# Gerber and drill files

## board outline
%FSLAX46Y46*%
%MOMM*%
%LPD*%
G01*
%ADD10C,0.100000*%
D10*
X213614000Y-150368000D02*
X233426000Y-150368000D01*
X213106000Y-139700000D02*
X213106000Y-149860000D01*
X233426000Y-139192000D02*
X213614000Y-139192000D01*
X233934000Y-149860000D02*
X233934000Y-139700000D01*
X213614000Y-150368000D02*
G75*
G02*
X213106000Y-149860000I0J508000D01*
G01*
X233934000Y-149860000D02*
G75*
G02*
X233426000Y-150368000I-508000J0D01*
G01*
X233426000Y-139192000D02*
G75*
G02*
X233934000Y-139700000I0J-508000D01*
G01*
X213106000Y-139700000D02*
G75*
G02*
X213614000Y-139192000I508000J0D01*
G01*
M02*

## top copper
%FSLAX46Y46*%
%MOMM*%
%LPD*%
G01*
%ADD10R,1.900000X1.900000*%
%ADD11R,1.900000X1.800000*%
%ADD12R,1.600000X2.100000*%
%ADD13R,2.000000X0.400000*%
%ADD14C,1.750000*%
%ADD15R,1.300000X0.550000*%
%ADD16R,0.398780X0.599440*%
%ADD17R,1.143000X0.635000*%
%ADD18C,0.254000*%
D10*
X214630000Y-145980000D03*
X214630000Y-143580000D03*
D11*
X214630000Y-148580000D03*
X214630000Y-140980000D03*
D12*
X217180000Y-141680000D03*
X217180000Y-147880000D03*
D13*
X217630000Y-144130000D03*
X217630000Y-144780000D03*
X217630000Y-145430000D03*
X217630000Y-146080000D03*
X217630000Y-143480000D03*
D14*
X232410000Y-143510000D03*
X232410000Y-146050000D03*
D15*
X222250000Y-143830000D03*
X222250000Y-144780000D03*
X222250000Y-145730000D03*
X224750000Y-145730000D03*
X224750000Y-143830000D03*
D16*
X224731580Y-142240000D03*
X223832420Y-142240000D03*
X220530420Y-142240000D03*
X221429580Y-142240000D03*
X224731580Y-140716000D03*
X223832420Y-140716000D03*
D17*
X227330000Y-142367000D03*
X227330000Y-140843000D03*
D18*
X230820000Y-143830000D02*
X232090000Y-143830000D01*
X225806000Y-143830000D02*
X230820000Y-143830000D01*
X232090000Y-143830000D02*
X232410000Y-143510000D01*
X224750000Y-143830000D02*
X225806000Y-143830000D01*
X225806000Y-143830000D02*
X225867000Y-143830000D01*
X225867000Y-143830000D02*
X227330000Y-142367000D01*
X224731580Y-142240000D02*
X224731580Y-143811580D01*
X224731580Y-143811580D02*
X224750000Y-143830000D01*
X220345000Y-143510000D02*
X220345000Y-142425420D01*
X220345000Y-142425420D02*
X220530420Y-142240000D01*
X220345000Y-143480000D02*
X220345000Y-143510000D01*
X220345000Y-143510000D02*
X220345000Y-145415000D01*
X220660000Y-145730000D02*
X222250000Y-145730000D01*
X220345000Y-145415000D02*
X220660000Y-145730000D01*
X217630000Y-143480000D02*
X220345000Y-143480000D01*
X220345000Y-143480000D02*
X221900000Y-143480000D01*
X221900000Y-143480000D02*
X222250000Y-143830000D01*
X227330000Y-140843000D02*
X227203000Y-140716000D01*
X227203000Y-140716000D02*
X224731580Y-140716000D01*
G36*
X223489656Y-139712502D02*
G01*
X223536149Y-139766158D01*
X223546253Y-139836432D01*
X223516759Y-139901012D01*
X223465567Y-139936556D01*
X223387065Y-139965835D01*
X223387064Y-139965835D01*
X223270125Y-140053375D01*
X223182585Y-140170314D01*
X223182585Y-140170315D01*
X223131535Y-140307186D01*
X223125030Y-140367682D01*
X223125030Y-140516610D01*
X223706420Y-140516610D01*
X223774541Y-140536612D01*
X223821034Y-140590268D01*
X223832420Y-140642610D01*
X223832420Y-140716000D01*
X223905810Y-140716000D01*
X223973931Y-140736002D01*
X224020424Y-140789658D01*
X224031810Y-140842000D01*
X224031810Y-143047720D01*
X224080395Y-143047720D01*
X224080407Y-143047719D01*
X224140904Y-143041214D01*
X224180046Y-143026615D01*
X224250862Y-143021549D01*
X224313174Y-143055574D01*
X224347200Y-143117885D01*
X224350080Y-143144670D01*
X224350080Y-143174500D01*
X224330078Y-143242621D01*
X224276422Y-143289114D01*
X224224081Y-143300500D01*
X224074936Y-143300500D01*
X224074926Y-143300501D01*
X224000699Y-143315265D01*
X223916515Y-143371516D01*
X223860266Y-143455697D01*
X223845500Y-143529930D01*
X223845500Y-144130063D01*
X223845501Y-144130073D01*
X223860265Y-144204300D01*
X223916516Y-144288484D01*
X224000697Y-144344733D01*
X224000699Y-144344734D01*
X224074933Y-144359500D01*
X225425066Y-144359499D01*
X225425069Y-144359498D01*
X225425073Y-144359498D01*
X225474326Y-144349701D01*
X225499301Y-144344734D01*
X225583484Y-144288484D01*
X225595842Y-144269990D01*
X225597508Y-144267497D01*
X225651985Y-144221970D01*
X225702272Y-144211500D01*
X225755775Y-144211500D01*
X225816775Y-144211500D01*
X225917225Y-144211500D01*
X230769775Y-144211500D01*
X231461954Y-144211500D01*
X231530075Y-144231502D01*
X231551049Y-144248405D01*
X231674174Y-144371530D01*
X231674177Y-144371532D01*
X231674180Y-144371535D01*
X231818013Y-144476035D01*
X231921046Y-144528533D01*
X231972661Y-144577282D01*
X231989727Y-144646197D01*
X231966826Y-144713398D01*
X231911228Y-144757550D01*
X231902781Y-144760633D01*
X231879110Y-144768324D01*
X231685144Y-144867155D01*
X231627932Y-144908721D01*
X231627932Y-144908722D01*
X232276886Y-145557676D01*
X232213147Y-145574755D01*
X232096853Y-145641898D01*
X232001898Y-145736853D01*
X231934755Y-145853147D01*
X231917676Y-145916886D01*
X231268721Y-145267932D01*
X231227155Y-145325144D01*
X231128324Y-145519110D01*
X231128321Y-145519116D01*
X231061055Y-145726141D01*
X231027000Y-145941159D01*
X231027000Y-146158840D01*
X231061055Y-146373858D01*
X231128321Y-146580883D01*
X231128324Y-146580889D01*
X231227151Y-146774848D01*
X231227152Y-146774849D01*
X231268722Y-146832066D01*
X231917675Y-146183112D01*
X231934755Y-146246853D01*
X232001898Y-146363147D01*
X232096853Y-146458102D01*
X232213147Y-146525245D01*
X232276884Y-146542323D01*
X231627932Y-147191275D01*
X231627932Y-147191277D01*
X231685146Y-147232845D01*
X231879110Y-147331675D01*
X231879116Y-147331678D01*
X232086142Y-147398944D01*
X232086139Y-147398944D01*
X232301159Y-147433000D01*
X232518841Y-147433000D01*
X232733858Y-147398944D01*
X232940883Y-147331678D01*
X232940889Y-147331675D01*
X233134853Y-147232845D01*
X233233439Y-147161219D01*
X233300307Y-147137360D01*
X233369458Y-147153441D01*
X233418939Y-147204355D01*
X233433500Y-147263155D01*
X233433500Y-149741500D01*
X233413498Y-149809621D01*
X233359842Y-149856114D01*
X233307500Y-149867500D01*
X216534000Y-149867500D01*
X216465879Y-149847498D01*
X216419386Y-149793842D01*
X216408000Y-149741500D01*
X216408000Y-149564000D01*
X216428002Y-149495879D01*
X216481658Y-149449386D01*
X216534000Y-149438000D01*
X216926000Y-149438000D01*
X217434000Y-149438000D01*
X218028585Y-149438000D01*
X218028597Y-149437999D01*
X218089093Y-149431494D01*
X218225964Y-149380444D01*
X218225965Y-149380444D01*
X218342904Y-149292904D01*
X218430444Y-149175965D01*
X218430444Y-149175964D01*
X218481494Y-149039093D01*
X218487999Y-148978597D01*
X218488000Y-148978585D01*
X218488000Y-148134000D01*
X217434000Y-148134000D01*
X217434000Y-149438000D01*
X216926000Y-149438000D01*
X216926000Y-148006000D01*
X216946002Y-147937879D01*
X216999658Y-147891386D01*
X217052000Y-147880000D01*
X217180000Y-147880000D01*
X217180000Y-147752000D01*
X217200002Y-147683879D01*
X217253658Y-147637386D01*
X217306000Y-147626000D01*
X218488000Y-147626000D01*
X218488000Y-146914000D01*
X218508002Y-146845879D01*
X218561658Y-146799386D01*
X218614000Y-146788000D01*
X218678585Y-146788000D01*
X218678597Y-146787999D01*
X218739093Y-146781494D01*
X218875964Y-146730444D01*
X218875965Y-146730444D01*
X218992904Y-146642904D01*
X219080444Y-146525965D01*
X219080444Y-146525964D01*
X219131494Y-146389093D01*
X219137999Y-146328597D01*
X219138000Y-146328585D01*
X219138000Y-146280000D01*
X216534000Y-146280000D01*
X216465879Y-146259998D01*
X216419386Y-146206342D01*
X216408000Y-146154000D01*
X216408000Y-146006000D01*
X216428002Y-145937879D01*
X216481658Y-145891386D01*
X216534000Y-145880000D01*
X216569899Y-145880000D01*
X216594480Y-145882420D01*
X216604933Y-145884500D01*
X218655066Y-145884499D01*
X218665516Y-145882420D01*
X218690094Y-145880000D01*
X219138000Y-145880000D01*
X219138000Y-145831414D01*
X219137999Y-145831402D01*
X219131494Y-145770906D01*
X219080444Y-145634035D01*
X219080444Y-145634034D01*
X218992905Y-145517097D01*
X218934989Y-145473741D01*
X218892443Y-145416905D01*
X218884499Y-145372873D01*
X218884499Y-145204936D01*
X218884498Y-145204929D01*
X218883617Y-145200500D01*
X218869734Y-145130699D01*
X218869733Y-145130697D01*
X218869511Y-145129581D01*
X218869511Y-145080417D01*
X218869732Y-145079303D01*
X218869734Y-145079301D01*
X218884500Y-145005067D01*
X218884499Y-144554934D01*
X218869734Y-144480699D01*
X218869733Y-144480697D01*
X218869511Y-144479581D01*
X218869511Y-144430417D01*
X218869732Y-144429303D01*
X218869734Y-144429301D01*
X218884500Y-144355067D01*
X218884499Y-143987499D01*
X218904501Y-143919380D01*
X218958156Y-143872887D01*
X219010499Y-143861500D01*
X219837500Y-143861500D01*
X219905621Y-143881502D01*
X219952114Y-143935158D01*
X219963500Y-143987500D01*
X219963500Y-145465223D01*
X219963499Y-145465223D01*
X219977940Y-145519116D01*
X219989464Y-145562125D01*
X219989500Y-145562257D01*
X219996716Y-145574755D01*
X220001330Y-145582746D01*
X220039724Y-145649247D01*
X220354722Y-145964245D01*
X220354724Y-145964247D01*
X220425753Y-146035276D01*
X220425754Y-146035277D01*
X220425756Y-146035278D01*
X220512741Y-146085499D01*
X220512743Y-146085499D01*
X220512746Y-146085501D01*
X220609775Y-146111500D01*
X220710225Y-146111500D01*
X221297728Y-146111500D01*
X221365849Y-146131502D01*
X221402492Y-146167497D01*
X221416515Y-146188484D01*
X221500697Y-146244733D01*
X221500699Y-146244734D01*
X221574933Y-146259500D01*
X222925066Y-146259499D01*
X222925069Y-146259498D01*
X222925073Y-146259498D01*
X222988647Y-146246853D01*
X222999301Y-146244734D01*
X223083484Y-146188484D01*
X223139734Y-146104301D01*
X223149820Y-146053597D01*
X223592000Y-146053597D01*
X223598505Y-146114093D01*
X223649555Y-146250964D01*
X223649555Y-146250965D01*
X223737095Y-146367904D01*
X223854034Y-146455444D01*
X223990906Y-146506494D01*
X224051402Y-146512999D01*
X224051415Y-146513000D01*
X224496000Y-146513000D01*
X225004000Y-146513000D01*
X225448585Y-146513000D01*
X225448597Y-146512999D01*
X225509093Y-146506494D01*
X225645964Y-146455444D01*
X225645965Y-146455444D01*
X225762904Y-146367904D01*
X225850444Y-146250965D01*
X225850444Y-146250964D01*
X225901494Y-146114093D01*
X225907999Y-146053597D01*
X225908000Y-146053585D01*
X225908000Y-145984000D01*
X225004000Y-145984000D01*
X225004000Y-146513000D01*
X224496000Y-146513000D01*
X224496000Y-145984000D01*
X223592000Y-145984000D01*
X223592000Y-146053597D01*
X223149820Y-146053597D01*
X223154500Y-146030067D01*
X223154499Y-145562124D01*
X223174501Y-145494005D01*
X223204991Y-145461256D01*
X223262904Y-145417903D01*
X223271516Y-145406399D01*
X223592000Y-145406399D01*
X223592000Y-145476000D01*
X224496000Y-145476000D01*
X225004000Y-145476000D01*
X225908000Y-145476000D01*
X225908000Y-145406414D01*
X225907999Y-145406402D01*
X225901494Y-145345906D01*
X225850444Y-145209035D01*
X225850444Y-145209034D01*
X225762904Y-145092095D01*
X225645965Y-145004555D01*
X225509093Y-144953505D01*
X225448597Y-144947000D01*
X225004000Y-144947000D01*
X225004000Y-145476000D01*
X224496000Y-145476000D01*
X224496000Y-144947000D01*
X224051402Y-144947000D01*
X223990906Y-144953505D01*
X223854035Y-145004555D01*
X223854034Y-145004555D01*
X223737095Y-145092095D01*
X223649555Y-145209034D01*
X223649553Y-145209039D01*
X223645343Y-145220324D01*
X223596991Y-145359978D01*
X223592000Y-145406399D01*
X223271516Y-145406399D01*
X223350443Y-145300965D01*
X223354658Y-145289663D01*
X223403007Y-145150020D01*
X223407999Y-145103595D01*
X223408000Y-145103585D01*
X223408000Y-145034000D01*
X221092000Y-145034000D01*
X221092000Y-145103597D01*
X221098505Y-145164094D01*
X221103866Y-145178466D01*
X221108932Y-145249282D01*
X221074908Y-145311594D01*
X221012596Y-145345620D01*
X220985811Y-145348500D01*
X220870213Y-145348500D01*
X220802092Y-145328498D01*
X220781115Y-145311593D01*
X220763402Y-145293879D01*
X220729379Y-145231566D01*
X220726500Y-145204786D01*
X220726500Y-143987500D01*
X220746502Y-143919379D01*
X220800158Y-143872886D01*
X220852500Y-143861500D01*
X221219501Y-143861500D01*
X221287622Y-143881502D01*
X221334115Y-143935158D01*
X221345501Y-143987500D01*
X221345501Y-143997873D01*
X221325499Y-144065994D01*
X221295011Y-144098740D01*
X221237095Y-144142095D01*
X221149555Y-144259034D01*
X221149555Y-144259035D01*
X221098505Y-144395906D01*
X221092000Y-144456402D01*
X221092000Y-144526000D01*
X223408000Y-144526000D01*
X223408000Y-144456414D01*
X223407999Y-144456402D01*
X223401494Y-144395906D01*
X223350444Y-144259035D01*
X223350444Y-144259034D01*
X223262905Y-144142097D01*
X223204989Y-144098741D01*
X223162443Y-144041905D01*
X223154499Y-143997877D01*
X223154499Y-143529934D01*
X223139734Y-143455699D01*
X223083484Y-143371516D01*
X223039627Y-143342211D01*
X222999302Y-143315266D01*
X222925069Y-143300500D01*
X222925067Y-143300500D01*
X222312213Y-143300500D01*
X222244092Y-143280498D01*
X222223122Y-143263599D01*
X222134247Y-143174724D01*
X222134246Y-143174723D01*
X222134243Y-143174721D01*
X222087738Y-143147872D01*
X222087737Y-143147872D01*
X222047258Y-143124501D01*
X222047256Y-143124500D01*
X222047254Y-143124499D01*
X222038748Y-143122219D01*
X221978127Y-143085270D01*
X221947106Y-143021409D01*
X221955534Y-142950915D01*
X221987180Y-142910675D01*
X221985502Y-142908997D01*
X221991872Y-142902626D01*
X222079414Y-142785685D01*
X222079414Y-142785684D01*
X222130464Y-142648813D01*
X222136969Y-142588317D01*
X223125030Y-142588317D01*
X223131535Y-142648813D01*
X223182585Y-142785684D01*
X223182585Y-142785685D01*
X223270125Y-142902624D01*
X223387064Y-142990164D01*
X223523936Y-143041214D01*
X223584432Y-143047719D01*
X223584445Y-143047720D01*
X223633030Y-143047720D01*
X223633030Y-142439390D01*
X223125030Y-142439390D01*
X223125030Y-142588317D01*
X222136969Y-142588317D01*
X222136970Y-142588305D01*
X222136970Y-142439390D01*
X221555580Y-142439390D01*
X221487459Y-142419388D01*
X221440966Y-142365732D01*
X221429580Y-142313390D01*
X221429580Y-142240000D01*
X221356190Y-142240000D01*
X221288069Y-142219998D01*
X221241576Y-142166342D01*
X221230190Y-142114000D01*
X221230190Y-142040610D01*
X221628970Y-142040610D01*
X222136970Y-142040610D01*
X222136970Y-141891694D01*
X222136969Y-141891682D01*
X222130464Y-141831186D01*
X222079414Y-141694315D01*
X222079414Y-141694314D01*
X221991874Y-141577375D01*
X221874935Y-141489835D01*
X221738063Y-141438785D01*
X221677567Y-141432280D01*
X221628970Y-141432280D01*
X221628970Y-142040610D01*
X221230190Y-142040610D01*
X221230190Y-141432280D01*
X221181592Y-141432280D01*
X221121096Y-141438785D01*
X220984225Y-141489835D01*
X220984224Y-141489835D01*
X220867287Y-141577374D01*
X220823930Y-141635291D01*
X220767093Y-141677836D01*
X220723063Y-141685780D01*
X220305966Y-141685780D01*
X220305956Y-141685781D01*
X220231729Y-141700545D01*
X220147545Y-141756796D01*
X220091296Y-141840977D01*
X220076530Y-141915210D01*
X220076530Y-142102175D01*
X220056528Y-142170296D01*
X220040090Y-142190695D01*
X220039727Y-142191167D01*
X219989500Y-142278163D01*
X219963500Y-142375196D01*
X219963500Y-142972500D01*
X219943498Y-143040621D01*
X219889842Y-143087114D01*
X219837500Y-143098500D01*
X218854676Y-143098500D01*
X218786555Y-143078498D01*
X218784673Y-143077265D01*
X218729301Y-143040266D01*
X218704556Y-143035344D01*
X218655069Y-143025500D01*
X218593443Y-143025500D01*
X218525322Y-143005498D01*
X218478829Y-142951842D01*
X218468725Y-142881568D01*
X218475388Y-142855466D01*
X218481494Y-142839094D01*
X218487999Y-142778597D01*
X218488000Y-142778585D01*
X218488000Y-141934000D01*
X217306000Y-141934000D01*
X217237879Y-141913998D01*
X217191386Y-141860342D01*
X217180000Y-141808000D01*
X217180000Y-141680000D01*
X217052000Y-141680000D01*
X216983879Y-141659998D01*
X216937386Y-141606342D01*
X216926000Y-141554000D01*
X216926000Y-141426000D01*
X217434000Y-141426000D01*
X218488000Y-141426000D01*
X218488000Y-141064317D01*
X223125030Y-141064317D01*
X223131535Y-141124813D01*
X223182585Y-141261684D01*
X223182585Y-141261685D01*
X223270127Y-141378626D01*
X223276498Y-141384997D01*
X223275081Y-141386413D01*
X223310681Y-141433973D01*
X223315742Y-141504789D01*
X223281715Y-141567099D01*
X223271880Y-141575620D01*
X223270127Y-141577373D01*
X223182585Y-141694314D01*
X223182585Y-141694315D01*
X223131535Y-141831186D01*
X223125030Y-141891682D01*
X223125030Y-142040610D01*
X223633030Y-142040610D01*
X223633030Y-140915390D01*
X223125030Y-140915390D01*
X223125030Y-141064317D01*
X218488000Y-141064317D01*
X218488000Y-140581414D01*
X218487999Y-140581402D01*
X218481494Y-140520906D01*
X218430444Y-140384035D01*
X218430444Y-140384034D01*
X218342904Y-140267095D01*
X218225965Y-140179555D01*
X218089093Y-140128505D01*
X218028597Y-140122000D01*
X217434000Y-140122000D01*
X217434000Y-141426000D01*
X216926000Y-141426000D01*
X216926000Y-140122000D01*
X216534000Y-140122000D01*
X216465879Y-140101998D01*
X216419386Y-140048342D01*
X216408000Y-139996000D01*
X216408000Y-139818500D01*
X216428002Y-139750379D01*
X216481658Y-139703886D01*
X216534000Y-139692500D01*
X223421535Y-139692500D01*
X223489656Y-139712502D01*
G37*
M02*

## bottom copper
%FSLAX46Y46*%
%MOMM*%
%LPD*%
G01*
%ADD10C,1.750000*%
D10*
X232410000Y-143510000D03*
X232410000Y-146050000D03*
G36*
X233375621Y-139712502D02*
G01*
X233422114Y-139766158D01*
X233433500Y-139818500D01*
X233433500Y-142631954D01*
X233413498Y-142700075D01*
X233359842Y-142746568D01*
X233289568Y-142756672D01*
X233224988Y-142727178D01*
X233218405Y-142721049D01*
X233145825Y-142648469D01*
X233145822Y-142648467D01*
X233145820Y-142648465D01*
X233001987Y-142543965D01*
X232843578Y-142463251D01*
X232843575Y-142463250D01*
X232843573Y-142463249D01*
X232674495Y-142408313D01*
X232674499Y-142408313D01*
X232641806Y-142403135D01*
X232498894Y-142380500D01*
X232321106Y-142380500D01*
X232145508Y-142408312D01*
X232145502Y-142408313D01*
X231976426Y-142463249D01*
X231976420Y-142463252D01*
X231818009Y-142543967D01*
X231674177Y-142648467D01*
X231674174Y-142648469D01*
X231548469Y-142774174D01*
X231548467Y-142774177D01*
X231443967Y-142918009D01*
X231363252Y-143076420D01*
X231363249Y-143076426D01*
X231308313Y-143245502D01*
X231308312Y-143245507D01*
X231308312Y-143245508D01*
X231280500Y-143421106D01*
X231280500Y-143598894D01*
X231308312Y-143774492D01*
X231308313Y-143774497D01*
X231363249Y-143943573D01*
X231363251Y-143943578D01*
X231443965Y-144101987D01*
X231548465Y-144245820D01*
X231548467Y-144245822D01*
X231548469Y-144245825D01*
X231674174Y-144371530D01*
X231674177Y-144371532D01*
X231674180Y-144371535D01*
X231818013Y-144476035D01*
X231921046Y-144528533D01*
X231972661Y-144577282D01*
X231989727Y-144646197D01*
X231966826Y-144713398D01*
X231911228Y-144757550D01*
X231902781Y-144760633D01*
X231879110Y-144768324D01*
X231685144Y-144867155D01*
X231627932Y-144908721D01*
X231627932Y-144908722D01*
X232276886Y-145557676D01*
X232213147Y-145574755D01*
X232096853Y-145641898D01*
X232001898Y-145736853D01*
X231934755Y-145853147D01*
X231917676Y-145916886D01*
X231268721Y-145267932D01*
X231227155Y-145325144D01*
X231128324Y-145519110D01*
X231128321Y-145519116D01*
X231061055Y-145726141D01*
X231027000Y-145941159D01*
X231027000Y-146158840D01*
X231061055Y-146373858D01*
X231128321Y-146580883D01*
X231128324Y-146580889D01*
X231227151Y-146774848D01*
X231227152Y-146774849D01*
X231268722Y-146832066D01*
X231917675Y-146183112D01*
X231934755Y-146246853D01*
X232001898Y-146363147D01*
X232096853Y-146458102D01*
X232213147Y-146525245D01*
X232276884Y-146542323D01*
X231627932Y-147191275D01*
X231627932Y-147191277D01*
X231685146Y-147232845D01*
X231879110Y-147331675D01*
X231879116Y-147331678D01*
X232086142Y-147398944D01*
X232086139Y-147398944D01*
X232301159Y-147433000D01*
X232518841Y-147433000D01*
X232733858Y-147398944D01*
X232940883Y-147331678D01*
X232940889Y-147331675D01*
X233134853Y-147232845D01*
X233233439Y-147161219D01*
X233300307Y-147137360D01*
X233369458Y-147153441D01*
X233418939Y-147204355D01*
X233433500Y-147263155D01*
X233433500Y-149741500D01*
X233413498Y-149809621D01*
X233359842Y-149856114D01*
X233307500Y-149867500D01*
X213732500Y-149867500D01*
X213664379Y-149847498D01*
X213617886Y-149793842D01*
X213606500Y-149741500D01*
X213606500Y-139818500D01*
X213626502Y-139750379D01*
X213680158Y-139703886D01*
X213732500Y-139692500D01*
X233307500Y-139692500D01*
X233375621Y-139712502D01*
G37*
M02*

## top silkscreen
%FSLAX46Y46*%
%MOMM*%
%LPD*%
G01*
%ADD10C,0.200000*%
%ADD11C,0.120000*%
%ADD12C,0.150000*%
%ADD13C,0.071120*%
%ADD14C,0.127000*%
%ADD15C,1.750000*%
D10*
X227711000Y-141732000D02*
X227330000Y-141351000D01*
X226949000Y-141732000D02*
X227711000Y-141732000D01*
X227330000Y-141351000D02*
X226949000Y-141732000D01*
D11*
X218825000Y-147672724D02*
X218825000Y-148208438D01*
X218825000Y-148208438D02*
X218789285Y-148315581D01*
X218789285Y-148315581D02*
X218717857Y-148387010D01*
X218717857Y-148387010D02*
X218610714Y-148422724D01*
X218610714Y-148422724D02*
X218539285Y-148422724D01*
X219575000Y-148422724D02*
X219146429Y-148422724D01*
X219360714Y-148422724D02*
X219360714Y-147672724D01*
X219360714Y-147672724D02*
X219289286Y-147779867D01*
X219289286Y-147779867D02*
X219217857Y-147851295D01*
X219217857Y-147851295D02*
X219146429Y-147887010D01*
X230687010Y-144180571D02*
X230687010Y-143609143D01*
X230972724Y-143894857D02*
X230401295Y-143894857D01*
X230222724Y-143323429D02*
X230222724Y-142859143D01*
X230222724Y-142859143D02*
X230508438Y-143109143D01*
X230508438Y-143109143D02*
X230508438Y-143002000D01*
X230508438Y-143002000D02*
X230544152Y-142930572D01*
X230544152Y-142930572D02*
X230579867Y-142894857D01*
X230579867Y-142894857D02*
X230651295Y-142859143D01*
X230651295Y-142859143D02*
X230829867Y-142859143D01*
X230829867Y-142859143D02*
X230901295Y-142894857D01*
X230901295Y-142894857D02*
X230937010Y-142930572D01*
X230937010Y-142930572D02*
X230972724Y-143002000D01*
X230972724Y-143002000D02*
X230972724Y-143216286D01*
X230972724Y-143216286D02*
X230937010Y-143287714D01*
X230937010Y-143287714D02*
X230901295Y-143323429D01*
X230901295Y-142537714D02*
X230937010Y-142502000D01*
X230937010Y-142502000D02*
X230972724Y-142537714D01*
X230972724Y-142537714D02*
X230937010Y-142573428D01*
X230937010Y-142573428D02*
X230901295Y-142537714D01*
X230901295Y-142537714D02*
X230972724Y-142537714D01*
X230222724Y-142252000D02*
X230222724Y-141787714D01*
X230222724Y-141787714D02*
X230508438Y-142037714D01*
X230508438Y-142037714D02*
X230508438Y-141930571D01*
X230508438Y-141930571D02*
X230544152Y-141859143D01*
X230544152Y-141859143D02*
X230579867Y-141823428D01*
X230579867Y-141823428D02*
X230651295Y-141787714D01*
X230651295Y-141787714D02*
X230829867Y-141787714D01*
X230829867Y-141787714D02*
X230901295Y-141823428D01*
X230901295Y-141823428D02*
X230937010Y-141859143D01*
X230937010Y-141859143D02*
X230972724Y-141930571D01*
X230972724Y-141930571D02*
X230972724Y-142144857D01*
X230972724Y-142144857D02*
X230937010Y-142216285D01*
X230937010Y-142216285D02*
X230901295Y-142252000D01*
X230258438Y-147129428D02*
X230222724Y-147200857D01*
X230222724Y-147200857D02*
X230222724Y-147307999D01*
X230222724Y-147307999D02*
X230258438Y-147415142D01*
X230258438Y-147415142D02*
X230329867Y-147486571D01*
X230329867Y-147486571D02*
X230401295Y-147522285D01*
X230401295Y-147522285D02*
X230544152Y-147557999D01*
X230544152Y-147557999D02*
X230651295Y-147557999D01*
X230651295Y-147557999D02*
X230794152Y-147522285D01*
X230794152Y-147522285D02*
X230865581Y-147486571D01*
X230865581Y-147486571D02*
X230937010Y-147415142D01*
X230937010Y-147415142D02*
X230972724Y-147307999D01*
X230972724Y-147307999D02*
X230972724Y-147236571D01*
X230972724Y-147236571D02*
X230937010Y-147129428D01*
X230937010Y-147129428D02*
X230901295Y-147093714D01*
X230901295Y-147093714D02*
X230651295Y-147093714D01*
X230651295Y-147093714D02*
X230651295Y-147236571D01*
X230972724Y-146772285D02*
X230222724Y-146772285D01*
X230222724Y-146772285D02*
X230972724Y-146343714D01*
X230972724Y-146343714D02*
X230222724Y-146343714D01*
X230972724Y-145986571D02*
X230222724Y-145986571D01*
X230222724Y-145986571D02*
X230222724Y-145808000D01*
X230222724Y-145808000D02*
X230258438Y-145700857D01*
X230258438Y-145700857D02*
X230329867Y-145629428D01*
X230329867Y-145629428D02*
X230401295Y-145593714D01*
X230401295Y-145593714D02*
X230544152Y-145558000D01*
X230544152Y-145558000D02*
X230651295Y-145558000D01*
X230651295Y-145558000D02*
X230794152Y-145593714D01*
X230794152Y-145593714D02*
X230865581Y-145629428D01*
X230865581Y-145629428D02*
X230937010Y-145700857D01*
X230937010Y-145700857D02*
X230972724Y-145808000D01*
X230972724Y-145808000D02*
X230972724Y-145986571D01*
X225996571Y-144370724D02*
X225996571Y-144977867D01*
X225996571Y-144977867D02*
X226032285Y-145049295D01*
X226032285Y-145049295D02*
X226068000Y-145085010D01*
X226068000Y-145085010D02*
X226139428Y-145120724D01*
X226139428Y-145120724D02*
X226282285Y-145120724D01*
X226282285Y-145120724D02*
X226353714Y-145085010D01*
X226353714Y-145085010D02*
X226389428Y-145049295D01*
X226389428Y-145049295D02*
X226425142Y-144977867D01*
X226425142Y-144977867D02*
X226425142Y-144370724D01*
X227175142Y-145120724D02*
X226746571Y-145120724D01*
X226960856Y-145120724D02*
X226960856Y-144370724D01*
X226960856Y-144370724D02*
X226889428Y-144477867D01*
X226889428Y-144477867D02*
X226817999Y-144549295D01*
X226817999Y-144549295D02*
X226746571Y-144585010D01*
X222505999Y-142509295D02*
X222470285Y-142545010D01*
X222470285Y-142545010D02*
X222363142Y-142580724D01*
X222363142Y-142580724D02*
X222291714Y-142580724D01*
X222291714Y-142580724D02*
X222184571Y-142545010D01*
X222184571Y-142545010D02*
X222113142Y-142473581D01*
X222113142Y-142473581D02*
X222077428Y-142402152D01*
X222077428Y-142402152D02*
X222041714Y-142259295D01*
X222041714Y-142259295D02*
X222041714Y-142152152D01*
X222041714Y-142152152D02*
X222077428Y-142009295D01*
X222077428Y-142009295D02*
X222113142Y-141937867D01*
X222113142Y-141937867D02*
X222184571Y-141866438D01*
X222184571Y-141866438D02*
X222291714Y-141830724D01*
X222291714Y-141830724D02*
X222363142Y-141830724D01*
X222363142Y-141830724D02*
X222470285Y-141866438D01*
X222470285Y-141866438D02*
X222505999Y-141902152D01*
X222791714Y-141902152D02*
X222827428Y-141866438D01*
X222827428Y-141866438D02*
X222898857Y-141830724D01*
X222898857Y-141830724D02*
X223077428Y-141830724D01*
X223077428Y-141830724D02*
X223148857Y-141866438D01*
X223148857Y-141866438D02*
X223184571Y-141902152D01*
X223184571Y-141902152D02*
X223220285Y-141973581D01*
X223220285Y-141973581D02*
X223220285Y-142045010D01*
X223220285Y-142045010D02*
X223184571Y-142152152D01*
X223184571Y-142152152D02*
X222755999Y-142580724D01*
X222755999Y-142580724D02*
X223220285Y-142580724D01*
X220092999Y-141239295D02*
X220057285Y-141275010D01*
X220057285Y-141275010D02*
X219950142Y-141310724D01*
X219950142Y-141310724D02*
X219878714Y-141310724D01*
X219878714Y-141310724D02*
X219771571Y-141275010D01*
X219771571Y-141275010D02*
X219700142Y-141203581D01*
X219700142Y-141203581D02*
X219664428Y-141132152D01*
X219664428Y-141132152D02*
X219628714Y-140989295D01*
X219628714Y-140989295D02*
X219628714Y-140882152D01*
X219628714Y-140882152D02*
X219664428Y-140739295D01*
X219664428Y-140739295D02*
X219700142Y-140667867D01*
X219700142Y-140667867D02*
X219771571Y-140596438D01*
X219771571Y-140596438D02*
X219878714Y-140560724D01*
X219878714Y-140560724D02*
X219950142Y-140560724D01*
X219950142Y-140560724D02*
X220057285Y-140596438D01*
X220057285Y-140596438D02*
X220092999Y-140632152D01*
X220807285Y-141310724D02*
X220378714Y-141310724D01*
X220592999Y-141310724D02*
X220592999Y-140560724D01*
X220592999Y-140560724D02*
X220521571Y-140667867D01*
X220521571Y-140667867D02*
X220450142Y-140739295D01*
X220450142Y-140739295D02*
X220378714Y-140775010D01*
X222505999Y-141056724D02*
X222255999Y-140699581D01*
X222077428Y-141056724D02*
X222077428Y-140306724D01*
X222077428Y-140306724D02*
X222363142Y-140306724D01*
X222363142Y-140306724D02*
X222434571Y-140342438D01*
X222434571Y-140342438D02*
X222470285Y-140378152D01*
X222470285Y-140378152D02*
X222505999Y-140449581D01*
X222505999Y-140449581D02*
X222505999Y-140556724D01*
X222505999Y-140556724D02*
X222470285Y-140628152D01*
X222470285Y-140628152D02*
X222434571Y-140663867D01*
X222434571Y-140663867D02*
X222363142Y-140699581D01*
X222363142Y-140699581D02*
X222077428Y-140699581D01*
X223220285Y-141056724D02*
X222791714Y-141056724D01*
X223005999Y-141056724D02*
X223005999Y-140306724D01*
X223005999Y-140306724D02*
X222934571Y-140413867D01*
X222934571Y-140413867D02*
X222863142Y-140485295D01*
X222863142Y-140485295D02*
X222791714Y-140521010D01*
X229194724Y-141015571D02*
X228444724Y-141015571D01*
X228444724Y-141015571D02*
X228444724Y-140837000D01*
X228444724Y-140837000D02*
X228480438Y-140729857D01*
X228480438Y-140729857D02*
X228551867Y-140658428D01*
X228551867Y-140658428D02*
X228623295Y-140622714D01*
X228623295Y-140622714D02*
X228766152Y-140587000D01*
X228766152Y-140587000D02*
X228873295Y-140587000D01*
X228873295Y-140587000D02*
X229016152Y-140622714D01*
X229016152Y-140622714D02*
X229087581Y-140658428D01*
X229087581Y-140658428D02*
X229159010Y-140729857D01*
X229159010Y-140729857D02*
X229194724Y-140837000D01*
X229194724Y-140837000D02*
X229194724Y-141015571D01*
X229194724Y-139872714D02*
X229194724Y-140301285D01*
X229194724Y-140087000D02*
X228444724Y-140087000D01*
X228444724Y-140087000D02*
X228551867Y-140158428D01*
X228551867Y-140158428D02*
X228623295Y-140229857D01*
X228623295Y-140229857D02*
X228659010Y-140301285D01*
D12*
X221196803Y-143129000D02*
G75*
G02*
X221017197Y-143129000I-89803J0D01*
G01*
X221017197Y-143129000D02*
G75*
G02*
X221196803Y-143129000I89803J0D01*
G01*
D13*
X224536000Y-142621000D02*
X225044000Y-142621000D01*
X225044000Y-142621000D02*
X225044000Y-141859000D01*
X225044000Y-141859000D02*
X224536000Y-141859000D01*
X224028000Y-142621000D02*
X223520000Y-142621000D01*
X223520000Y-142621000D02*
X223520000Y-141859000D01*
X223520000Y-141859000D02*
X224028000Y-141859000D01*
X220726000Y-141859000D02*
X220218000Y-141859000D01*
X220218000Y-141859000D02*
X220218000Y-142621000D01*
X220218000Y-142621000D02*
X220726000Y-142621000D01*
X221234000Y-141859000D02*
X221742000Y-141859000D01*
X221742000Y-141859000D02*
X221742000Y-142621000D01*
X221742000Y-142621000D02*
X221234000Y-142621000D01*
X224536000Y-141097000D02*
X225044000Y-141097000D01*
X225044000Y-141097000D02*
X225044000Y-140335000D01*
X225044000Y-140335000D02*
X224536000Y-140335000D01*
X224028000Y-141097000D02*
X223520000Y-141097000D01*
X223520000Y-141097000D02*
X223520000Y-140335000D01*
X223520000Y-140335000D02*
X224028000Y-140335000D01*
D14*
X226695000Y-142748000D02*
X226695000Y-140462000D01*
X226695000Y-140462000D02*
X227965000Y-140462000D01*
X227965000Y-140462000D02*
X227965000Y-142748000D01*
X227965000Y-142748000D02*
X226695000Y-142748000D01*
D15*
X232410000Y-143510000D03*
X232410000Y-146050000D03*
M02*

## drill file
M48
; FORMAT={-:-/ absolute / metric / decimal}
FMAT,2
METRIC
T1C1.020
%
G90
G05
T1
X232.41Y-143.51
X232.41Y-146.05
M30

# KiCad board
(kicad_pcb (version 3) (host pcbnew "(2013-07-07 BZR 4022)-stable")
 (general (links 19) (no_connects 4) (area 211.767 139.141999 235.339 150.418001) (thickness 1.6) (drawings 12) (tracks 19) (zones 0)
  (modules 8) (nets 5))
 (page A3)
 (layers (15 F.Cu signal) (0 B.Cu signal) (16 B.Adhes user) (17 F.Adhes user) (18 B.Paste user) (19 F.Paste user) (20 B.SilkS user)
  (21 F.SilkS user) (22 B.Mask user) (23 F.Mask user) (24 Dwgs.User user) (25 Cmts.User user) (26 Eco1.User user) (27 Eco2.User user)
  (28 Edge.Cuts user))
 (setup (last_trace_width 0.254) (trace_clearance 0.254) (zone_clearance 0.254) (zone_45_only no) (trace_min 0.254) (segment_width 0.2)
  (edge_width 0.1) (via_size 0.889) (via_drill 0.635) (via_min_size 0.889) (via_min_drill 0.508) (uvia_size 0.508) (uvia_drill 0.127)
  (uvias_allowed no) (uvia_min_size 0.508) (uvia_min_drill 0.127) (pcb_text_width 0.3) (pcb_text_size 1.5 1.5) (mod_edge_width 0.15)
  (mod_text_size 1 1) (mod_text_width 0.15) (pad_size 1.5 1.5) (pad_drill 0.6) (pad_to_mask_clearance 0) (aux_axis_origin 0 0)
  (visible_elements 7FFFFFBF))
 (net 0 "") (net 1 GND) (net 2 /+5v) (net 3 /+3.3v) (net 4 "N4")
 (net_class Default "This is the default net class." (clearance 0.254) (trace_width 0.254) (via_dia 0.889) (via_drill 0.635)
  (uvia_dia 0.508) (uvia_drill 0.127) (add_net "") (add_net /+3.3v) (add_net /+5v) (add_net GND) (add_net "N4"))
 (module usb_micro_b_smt (layer F.Cu) (at 214.63 144.78 270)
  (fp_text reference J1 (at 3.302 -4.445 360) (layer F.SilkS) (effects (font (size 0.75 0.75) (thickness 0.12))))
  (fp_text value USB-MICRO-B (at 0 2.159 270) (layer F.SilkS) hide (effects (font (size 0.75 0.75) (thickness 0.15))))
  (pad 6 smd rect (at 1.2 0 270) (size 1.9 1.9) (layers F.Cu F.Paste F.Mask) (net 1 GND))
  (pad 6 smd rect (at -1.2 0 270) (size 1.9 1.9) (layers F.Cu F.Paste F.Mask) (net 1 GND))
  (pad 6 smd rect (at 3.8 0 270) (size 1.8 1.9) (layers F.Cu F.Paste F.Mask) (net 1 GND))
  (pad 6 smd rect (at -3.8 0 270) (size 1.8 1.9) (layers F.Cu F.Paste F.Mask) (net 1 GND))
  (pad 6 smd rect (at -3.1 -2.55 270) (size 2.1 1.6) (layers F.Cu F.Paste F.Mask) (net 1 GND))
  (pad 6 smd rect (at 3.1 -2.55 270) (size 2.1 1.6) (layers F.Cu F.Paste F.Mask) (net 1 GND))
  (pad 2 smd rect (at -0.65 -3 270) (size 0.4 2) (layers F.Cu F.Paste F.Mask))
  (pad 3 smd rect (at 0 -3 270) (size 0.4 2) (layers F.Cu F.Paste F.Mask))
  (pad 4 smd rect (at 0.65 -3 270) (size 0.4 2) (layers F.Cu F.Paste F.Mask))
  (pad 5 smd rect (at 1.3 -3 270) (size 0.4 2) (layers F.Cu F.Paste F.Mask) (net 1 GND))
  (pad 1 smd rect (at -1.3 -3 270) (size 0.4 2) (layers F.Cu F.Paste F.Mask) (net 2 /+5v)))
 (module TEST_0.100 (layer F.Cu) (at 232.41 143.51 270)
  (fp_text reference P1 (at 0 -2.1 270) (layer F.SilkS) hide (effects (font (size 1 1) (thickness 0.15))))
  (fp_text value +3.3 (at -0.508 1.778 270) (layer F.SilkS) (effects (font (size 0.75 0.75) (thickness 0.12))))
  (pad 1 thru_hole circle (at 0 0 270) (size 1.75 1.75) (drill 1.02) (layers *.Cu *.Mask F.SilkS) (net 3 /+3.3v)))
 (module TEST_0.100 (layer F.Cu) (at 232.41 146.05 270)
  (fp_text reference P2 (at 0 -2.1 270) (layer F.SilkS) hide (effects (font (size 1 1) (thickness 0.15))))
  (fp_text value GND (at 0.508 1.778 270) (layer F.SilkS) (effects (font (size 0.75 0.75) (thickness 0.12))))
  (pad 1 thru_hole circle (at 0 0 270) (size 1.75 1.75) (drill 1.02) (layers *.Cu *.Mask F.SilkS) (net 1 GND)))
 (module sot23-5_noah (layer F.Cu) (at 222.25 144.78)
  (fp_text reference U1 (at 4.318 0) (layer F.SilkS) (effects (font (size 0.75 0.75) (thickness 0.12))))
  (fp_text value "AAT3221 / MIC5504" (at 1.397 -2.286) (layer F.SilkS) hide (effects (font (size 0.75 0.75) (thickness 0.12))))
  (fp_circle (center -1.143 -1.651) (end -1.0795 -1.5875) (layer F.SilkS) (width 0.15))
  (pad 1 smd rect (at 0 -0.95) (size 1.3 0.55) (layers F.Cu F.Paste F.Mask) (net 2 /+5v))
  (pad 2 smd rect (at 0 0) (size 1.3 0.55) (layers F.Cu F.Paste F.Mask) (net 1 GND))
  (pad 3 smd rect (at 0 0.95) (size 1.3 0.55) (layers F.Cu F.Paste F.Mask) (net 2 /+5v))
  (pad 4 smd rect (at 2.5 0.95) (size 1.3 0.55) (layers F.Cu F.Paste F.Mask) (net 1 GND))
  (pad 5 smd rect (at 2.5 -0.95) (size 1.3 0.55) (layers F.Cu F.Paste F.Mask) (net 3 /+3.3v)))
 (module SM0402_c (layer F.Cu) (at 224.282 142.24 180)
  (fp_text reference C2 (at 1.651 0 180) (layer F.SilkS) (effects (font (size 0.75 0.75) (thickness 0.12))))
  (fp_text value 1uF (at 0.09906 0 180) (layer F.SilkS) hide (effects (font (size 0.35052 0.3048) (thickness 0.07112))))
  (fp_line (start -0.254 -0.381) (end -0.762 -0.381) (layer F.SilkS) (width 0.07112))
  (fp_line (start -0.762 -0.381) (end -0.762 0.381) (layer F.SilkS) (width 0.07112))
  (fp_line (start -0.762 0.381) (end -0.254 0.381) (layer F.SilkS) (width 0.07112))
  (fp_line (start 0.254 -0.381) (end 0.762 -0.381) (layer F.SilkS) (width 0.07112))
  (fp_line (start 0.762 -0.381) (end 0.762 0.381) (layer F.SilkS) (width 0.07112))
  (fp_line (start 0.762 0.381) (end 0.254 0.381) (layer F.SilkS) (width 0.07112))
  (pad 1 smd rect (at -0.44958 0 180) (size 0.39878 0.59944) (layers F.Cu F.Paste F.Mask) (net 3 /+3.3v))
  (pad 2 smd rect (at 0.44958 0 180) (size 0.39878 0.59944) (layers F.Cu F.Paste F.Mask) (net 1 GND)))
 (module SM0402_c (layer F.Cu) (at 220.98 142.24)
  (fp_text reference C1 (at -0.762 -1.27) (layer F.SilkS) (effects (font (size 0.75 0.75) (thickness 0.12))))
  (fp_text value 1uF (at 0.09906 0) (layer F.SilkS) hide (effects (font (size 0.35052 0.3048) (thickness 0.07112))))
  (fp_line (start -0.254 -0.381) (end -0.762 -0.381) (layer F.SilkS) (width 0.07112))
  (fp_line (start -0.762 -0.381) (end -0.762 0.381) (layer F.SilkS) (width 0.07112))
  (fp_line (start -0.762 0.381) (end -0.254 0.381) (layer F.SilkS) (width 0.07112))
  (fp_line (start 0.254 -0.381) (end 0.762 -0.381) (layer F.SilkS) (width 0.07112))
  (fp_line (start 0.762 -0.381) (end 0.762 0.381) (layer F.SilkS) (width 0.07112))
  (fp_line (start 0.762 0.381) (end 0.254 0.381) (layer F.SilkS) (width 0.07112))
  (pad 1 smd rect (at -0.44958 0) (size 0.39878 0.59944) (layers F.Cu F.Paste F.Mask) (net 2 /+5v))
  (pad 2 smd rect (at 0.44958 0) (size 0.39878 0.59944) (layers F.Cu F.Paste F.Mask) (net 1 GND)))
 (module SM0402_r (layer F.Cu) (at 224.282 140.716 180)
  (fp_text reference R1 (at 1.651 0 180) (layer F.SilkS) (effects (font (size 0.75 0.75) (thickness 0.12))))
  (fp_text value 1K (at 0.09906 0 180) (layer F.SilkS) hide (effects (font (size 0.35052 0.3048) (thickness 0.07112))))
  (fp_line (start -0.254 -0.381) (end -0.762 -0.381) (layer F.SilkS) (width 0.07112))
  (fp_line (start -0.762 -0.381) (end -0.762 0.381) (layer F.SilkS) (width 0.07112))
  (fp_line (start -0.762 0.381) (end -0.254 0.381) (layer F.SilkS) (width 0.07112))
  (fp_line (start 0.254 -0.381) (end 0.762 -0.381) (layer F.SilkS) (width 0.07112))
  (fp_line (start 0.762 -0.381) (end 0.762 0.381) (layer F.SilkS) (width 0.07112))
  (fp_line (start 0.762 0.381) (end 0.254 0.381) (layer F.SilkS) (width 0.07112))
  (pad 1 smd rect (at -0.44958 0 180) (size 0.39878 0.59944) (layers F.Cu F.Paste F.Mask) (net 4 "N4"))
  (pad 2 smd rect (at 0.44958 0 180) (size 0.39878 0.59944) (layers F.Cu F.Paste F.Mask) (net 1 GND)))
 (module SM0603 (layer F.Cu) (at 227.33 141.605 90)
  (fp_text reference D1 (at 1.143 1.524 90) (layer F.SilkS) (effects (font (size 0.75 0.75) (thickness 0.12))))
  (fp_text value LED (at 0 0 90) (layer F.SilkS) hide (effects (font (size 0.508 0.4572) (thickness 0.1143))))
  (fp_line (start -1.143 -0.635) (end 1.143 -0.635) (layer F.SilkS) (width 0.127))
  (fp_line (start 1.143 -0.635) (end 1.143 0.635) (layer F.SilkS) (width 0.127))
  (fp_line (start 1.143 0.635) (end -1.143 0.635) (layer F.SilkS) (width 0.127))
  (fp_line (start -1.143 0.635) (end -1.143 -0.635) (layer F.SilkS) (width 0.127))
  (pad 1 smd rect (at -0.762 0 90) (size 0.635 1.143) (layers F.Cu F.Paste F.Mask) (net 3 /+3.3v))
  (pad 2 smd rect (at 0.762 0 90) (size 0.635 1.143) (layers F.Cu F.Paste F.Mask) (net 4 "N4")))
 (gr_line (start 227.711 141.732) (end 227.33 141.351) (angle 90) (layer F.SilkS) (width 0.2))
 (gr_line (start 226.949 141.732) (end 227.711 141.732) (angle 90) (layer F.SilkS) (width 0.2))
 (gr_line (start 227.33 141.351) (end 226.949 141.732) (angle 90) (layer F.SilkS) (width 0.2))
 (gr_line (start 213.614 150.368) (end 233.426 150.368) (angle 90) (layer Edge.Cuts) (width 0.1))
 (gr_line (start 213.106 139.7) (end 213.106 149.86) (angle 90) (layer Edge.Cuts) (width 0.1))
 (gr_line (start 233.426 139.192) (end 213.614 139.192) (angle 90) (layer Edge.Cuts) (width 0.1))
 (gr_line (start 233.934 149.86) (end 233.934 139.7) (angle 90) (layer Edge.Cuts) (width 0.1))
 (gr_arc (start 213.614 149.86) (end 213.614 150.368) (angle 90) (layer Edge.Cuts) (width 0.1))
 (gr_arc (start 233.426 149.86) (end 233.934 149.86) (angle 90) (layer Edge.Cuts) (width 0.1))
 (gr_arc (start 233.426 139.7) (end 233.426 139.192) (angle 90) (layer Edge.Cuts) (width 0.1))
 (gr_arc (start 213.614 139.7) (end 213.106 139.7) (angle 90) (layer Edge.Cuts) (width 0.1))
 (segment (start 230.82 143.83) (end 232.09 143.83) (width 0.254) (layer F.Cu) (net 3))
 (segment (start 225.806 143.83) (end 230.82 143.83) (width 0.254) (layer F.Cu) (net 3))
 (segment (start 232.09 143.83) (end 232.41 143.51) (width 0.254) (layer F.Cu) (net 3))
 (segment (start 224.75 143.83) (end 225.806 143.83) (width 0.254) (layer F.Cu) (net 3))
 (segment (start 225.806 143.83) (end 225.867 143.83) (width 0.254) (layer F.Cu) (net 3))
 (segment (start 225.867 143.83) (end 227.33 142.367) (width 0.254) (layer F.Cu) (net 3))
 (segment (start 224.73158 142.24) (end 224.73158 143.81158) (width 0.254) (layer F.Cu) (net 3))
 (segment (start 224.73158 143.81158) (end 224.75 143.83) (width 0.254) (layer F.Cu) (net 3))
 (segment (start 220.345 143.51) (end 220.345 142.42542) (width 0.254) (layer F.Cu) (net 2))
 (segment (start 220.345 142.42542) (end 220.53042 142.24) (width 0.254) (layer F.Cu) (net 2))
 (segment (start 220.345 143.48) (end 220.345 143.51) (width 0.254) (layer F.Cu) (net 2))
 (segment (start 220.345 143.51) (end 220.345 145.415) (width 0.254) (layer F.Cu) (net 2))
 (segment (start 220.66 145.73) (end 222.25 145.73) (width 0.254) (layer F.Cu) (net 2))
 (segment (start 220.345 145.415) (end 220.66 145.73) (width 0.254) (layer F.Cu) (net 2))
 (segment (start 217.63 143.48) (end 220.345 143.48) (width 0.254) (layer F.Cu) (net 2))
 (segment (start 220.345 143.48) (end 221.9 143.48) (width 0.254) (layer F.Cu) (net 2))
 (segment (start 221.9 143.48) (end 222.25 143.83) (width 0.254) (layer F.Cu) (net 2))
 (segment (start 227.33 140.843) (end 227.203 140.716) (width 0.254) (layer F.Cu) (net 4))
 (segment (start 227.203 140.716) (end 224.73158 140.716) (width 0.254) (layer F.Cu) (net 4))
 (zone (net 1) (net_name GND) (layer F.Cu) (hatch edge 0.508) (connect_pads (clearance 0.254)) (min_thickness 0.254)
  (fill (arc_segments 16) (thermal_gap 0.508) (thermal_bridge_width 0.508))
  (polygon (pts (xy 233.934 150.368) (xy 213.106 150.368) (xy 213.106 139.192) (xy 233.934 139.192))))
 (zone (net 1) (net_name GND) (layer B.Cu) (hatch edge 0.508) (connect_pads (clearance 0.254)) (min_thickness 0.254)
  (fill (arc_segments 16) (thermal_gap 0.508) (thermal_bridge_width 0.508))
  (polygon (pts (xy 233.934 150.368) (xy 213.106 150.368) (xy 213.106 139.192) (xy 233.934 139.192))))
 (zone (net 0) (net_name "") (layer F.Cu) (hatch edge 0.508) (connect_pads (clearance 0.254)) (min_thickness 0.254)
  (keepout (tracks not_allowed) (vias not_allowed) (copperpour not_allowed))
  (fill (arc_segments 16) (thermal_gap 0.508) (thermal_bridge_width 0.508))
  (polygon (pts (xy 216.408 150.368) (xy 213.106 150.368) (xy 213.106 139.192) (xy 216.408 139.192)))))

